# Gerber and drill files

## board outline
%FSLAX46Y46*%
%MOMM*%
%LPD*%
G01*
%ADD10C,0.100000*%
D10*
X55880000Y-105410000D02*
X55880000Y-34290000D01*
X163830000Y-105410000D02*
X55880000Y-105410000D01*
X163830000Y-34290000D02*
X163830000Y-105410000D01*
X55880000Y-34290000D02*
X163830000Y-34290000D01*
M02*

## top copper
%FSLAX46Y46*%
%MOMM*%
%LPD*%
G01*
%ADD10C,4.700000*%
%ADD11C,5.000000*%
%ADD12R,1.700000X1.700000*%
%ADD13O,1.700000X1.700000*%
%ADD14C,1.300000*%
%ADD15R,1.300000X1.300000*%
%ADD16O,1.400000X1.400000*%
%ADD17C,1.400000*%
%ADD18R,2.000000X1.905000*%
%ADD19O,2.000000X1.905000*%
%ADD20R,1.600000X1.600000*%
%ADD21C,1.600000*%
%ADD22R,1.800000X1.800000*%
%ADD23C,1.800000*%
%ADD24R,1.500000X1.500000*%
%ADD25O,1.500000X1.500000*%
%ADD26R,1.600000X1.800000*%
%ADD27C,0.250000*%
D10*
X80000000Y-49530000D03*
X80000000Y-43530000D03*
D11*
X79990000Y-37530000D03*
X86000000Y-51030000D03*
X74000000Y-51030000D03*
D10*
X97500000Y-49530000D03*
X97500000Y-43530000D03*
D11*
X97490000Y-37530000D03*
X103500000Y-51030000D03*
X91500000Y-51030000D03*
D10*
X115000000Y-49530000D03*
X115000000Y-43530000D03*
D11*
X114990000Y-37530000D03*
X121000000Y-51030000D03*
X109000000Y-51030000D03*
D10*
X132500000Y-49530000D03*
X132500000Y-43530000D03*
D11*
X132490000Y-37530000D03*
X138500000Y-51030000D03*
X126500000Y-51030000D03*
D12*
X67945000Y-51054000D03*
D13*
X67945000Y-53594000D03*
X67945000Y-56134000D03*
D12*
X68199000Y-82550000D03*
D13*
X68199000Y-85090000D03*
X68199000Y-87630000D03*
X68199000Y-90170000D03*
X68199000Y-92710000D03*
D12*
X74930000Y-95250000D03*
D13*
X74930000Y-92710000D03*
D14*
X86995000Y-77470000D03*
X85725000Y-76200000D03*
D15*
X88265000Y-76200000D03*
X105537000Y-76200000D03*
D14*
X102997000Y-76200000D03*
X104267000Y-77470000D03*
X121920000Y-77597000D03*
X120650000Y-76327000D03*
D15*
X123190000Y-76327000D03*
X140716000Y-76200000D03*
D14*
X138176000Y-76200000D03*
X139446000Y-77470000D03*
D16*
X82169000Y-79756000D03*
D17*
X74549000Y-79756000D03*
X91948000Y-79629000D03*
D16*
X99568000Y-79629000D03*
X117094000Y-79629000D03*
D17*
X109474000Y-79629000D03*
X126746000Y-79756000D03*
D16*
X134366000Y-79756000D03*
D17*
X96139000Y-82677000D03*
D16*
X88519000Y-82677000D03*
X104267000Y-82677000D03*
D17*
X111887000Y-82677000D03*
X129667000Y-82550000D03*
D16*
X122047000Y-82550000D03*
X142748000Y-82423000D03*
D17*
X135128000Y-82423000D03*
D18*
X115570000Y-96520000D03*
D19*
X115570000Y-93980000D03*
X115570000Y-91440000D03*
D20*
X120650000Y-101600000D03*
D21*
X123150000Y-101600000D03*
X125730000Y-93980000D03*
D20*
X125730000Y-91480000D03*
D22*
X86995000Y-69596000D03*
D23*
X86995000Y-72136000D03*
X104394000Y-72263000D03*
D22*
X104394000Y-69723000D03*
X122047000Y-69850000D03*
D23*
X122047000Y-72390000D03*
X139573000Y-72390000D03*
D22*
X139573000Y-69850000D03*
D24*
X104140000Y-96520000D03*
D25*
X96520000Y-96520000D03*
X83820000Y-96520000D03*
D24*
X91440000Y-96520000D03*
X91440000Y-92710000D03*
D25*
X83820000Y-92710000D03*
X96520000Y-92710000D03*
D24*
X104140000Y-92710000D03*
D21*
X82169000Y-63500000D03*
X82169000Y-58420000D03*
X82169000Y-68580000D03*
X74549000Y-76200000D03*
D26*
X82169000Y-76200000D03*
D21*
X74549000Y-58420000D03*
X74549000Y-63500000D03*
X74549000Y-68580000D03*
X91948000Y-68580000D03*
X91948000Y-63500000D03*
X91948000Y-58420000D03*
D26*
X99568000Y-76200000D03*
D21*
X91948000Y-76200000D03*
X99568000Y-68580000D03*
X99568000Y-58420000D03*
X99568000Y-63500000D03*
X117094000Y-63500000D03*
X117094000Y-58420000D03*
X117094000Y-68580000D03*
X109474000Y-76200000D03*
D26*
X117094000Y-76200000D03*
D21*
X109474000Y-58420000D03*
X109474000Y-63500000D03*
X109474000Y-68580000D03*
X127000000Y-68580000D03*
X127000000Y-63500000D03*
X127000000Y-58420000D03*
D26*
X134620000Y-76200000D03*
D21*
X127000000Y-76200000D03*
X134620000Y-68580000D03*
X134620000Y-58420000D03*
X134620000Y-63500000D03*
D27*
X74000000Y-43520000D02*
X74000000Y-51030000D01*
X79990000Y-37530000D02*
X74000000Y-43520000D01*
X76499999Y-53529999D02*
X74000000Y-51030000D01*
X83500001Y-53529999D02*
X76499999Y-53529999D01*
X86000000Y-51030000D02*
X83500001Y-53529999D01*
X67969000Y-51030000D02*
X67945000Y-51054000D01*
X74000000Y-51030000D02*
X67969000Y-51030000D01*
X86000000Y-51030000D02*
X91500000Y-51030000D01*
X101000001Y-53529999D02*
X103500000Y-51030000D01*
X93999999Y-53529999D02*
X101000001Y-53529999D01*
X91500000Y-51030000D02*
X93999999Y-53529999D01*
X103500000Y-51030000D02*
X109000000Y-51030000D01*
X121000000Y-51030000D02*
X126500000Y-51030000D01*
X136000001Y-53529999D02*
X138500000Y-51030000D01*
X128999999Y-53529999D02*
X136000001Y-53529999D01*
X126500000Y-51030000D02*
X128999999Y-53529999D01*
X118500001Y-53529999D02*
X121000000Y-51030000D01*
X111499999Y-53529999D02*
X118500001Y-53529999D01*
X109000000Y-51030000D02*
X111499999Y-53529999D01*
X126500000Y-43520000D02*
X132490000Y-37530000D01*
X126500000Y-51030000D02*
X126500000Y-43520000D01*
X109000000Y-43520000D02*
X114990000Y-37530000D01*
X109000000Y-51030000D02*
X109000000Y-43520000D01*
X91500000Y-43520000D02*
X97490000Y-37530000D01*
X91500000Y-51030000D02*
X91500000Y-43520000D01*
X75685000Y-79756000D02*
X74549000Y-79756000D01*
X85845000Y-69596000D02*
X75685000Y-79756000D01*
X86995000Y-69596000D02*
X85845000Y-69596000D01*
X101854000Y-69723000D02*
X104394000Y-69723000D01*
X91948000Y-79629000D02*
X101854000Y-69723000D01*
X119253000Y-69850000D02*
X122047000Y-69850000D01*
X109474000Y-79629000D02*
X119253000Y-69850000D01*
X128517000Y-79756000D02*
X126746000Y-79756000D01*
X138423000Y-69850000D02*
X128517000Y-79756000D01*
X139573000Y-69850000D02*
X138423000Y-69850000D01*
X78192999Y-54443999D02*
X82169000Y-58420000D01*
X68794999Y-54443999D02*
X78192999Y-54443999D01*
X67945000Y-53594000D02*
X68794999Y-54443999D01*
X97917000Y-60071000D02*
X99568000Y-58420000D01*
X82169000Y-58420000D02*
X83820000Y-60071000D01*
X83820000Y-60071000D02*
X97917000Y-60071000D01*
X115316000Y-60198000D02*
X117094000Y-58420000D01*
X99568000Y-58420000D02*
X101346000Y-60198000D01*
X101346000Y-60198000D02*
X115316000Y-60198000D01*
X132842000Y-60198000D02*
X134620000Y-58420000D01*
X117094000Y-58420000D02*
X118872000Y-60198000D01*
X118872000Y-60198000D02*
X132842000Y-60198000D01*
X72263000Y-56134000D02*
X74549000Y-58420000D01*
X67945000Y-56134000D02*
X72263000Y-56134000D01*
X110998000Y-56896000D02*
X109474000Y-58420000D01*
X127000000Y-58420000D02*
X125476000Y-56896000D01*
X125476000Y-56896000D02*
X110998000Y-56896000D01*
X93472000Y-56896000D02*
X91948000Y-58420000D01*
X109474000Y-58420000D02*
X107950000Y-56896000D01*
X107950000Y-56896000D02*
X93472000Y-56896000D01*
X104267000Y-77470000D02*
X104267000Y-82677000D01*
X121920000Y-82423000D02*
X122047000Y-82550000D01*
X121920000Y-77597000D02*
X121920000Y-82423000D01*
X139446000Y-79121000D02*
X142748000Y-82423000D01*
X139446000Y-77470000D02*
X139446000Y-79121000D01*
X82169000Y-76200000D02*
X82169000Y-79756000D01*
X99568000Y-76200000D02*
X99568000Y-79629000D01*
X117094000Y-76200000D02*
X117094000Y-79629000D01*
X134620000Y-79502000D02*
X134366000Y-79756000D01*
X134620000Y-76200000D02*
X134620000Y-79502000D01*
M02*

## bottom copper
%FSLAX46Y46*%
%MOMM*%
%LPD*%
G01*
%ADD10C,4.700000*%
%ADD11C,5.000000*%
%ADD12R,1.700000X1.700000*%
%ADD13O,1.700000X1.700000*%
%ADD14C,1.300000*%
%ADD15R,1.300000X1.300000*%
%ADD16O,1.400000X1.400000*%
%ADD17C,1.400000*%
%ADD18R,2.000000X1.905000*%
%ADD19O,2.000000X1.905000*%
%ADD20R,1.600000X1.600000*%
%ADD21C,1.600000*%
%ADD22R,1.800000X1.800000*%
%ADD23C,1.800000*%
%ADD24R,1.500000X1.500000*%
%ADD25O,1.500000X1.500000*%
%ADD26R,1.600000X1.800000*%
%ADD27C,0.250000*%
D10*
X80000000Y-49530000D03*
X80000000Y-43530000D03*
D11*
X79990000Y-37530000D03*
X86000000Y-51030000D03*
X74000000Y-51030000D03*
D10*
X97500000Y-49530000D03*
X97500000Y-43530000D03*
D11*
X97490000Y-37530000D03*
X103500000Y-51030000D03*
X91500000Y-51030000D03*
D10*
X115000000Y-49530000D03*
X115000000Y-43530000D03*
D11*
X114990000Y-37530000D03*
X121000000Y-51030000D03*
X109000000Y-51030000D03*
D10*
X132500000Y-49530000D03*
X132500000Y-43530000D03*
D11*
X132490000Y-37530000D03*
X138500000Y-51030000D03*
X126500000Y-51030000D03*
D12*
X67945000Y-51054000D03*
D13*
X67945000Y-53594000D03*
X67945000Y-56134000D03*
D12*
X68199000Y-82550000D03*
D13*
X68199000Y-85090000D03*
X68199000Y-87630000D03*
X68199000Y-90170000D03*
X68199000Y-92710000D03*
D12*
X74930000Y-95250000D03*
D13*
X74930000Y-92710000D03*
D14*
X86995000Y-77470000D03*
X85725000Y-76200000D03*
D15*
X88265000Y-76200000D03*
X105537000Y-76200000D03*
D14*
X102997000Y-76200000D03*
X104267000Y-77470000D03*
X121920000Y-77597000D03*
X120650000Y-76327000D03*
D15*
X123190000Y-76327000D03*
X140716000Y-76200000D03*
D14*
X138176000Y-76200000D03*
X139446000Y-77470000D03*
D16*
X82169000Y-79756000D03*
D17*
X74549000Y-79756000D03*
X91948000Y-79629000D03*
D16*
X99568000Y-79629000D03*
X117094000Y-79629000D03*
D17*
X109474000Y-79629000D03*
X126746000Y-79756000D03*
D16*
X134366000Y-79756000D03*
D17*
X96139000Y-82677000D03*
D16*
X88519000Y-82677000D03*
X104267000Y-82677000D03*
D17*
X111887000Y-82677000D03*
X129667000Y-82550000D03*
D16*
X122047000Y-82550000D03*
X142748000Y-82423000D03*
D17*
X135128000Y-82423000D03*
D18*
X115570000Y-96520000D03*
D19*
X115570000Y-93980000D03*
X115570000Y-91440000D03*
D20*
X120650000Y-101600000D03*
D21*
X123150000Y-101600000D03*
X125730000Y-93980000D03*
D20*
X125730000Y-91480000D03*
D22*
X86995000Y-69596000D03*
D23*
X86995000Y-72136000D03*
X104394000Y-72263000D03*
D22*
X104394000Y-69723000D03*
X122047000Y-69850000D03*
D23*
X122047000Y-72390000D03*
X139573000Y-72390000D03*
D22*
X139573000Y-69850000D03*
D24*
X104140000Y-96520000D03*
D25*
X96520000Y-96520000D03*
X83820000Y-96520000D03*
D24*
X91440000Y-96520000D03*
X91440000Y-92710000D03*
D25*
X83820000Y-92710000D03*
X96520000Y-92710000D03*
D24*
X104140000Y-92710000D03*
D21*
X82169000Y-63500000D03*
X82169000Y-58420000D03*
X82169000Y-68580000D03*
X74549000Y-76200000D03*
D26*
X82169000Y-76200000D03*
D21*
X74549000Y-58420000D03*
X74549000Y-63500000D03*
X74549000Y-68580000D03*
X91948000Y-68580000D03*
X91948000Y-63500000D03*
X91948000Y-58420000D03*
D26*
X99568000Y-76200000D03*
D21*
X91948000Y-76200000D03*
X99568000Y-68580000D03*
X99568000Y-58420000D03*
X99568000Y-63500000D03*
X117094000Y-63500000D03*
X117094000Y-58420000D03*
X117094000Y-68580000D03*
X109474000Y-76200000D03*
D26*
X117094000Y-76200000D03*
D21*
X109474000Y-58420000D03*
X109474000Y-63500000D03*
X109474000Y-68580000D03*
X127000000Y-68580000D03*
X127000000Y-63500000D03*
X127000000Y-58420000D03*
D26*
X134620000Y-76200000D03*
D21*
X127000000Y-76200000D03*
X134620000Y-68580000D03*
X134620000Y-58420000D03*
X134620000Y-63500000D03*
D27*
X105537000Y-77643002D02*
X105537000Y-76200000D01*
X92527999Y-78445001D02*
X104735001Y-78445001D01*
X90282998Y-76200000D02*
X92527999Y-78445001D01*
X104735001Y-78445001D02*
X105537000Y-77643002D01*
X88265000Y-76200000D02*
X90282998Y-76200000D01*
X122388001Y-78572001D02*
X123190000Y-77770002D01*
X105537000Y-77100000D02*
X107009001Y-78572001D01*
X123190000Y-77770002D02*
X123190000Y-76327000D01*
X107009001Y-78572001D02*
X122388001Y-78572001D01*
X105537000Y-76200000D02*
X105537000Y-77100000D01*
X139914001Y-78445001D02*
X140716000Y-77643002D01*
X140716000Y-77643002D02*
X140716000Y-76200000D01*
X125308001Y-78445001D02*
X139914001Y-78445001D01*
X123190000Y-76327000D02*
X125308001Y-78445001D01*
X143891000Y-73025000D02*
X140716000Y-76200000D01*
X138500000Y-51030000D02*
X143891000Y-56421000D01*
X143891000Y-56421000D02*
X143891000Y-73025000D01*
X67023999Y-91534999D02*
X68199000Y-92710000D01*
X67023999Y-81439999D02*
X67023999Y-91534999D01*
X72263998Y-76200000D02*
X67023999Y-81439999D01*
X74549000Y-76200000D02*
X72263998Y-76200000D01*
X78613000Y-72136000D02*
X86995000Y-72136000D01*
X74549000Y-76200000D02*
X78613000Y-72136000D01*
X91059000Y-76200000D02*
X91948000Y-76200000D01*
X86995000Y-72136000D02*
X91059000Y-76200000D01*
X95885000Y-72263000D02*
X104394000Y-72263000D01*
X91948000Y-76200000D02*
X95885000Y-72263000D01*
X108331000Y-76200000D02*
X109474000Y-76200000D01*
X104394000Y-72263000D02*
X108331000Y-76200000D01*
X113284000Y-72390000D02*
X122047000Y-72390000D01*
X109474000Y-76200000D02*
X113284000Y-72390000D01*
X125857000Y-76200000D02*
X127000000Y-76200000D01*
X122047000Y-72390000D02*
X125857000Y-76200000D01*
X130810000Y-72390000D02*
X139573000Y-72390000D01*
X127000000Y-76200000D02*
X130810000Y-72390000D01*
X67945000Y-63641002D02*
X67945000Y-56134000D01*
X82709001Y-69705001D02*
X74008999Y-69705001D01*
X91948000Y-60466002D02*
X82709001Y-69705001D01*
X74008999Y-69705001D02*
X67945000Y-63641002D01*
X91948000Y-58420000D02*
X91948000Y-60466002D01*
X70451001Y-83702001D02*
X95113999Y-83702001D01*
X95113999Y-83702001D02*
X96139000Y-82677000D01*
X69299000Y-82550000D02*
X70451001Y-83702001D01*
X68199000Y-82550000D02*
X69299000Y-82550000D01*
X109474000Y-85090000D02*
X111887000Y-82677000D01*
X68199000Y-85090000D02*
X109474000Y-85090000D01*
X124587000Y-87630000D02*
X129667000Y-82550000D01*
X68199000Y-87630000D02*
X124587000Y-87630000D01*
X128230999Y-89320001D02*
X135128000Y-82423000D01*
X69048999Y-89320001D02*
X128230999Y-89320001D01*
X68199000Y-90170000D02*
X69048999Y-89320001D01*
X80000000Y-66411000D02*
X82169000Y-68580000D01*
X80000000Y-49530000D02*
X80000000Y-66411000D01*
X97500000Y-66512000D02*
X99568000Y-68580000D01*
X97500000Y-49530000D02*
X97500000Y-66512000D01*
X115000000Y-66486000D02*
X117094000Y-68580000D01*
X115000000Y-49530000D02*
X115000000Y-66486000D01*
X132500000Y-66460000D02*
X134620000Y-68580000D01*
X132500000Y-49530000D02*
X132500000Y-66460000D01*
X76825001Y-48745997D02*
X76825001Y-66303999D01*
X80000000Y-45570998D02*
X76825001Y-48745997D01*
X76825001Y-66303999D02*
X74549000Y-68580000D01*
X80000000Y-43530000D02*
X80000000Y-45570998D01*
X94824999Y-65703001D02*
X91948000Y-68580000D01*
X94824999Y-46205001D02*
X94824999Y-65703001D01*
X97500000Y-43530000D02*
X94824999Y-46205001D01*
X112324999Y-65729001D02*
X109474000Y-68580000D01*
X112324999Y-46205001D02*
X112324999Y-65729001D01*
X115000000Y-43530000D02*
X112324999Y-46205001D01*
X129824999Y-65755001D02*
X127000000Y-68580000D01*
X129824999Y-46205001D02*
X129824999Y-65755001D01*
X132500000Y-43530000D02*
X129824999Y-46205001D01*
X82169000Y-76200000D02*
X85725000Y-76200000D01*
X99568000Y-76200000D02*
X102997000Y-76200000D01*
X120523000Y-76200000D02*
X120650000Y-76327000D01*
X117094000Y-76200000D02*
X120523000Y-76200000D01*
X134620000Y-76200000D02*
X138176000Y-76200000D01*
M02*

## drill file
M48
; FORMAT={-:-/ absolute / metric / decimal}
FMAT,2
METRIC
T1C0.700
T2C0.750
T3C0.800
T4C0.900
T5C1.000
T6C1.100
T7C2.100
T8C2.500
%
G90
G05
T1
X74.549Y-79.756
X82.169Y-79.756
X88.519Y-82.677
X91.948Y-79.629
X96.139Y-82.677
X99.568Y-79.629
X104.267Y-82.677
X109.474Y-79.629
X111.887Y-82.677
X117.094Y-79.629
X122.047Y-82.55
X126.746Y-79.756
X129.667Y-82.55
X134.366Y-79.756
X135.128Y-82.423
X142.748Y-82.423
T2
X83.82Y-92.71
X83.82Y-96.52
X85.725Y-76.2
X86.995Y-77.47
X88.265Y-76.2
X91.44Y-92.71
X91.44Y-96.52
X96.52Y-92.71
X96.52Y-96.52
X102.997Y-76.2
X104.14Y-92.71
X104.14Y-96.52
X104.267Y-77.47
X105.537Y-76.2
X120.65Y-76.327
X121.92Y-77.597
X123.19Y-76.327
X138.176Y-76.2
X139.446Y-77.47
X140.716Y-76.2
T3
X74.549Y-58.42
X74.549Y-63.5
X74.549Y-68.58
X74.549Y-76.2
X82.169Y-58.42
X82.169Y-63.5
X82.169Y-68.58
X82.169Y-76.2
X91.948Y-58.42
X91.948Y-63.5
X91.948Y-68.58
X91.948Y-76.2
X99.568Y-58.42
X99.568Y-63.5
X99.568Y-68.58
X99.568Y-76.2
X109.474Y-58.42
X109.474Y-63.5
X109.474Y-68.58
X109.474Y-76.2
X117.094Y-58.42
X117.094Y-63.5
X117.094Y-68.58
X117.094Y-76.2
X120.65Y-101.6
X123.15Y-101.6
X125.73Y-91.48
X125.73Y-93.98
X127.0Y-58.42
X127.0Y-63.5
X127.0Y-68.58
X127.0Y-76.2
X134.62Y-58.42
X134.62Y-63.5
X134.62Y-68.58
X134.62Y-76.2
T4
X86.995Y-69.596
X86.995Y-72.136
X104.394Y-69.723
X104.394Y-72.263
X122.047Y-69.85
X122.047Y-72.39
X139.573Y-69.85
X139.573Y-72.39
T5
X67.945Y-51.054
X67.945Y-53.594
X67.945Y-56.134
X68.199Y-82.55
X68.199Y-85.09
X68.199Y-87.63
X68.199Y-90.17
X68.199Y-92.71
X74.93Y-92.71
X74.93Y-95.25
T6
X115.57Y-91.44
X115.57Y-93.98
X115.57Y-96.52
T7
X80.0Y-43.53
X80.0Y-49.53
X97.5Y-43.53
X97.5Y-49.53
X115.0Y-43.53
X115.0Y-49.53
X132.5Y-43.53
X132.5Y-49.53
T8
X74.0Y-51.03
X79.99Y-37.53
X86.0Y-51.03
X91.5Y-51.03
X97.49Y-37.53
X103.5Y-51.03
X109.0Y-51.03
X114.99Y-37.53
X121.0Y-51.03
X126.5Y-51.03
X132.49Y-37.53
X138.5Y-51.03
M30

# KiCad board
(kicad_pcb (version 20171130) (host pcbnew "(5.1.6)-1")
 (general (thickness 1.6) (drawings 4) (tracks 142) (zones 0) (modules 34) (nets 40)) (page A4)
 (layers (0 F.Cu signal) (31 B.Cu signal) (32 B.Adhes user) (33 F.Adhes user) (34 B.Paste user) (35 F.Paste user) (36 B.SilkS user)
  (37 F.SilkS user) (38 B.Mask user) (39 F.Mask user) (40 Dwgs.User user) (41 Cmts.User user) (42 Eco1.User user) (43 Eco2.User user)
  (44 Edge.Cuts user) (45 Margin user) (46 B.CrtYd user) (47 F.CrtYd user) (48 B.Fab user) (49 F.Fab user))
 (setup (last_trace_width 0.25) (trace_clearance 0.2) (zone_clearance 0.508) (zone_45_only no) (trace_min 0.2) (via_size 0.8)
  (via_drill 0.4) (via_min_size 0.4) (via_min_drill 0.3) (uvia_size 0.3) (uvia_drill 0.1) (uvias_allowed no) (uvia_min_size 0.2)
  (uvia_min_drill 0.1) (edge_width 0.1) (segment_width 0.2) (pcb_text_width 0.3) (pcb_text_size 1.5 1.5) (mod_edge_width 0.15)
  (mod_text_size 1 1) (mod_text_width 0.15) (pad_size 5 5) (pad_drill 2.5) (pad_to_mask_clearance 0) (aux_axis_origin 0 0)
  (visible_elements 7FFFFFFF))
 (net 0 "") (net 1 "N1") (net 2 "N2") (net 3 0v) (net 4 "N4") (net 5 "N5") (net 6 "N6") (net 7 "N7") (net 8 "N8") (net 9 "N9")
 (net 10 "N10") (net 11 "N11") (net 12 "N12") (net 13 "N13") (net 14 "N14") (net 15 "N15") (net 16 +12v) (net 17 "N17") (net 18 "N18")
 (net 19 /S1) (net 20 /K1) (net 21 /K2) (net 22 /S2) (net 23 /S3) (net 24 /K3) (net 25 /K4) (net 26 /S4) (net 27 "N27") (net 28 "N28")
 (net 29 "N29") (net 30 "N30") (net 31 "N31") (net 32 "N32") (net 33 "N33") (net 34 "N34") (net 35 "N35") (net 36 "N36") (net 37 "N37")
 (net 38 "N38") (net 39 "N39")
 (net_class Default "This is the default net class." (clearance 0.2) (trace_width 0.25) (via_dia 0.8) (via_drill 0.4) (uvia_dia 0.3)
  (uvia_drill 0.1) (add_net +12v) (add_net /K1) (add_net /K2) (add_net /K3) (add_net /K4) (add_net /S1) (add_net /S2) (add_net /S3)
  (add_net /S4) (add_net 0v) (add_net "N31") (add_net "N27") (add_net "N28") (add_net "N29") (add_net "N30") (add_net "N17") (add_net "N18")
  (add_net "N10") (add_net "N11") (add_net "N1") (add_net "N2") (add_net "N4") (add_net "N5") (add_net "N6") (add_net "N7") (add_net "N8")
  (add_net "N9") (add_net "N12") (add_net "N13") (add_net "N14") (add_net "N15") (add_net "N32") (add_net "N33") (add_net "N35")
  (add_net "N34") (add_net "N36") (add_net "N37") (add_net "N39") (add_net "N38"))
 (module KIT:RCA (layer F.Cu) (at 80 49.53 270)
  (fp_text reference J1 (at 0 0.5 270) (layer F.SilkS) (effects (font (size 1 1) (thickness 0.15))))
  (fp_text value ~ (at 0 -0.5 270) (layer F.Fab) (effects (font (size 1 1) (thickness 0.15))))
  (pad 1 thru_hole circle (at 0 0 270) (size 4.7 4.7) (drill 2.1) (layers *.Cu *.Mask) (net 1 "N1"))
  (pad 3 thru_hole circle (at -6 0 270) (size 4.7 4.7) (drill 2.1) (layers *.Cu *.Mask) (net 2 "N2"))
  (pad 2 thru_hole circle (at -12 0.01 270) (size 5 5) (drill 2.5) (layers *.Cu *.Mask) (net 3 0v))
  (pad 2 thru_hole circle (at 1.5 -6 270) (size 5 5) (drill 2.5) (layers *.Cu *.Mask) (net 3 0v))
  (pad 2 thru_hole circle (at 1.5 6 270) (size 5 5) (drill 2.5) (layers *.Cu *.Mask) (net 3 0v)))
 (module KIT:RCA (layer F.Cu) (at 97.5 49.53 270)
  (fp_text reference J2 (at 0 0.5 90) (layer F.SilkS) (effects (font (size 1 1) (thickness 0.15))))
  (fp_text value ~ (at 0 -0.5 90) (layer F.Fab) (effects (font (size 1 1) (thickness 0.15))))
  (pad 1 thru_hole circle (at 0 0 270) (size 4.7 4.7) (drill 2.1) (layers *.Cu *.Mask) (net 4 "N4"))
  (pad 3 thru_hole circle (at -6 0 270) (size 4.7 4.7) (drill 2.1) (layers *.Cu *.Mask) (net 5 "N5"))
  (pad 2 thru_hole circle (at -12 0.01 270) (size 5 5) (drill 2.5) (layers *.Cu *.Mask) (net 3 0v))
  (pad 2 thru_hole circle (at 1.5 -6 270) (size 5 5) (drill 2.5) (layers *.Cu *.Mask) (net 3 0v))
  (pad 2 thru_hole circle (at 1.5 6 270) (size 5 5) (drill 2.5) (layers *.Cu *.Mask) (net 3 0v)))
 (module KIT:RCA (layer F.Cu) (at 115 49.53 270)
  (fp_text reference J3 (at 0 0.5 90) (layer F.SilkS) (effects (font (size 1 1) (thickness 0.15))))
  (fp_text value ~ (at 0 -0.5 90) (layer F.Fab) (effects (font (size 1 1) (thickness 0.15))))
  (pad 1 thru_hole circle (at 0 0 270) (size 4.7 4.7) (drill 2.1) (layers *.Cu *.Mask) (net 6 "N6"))
  (pad 3 thru_hole circle (at -6 0 270) (size 4.7 4.7) (drill 2.1) (layers *.Cu *.Mask) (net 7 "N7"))
  (pad 2 thru_hole circle (at -12 0.01 270) (size 5 5) (drill 2.5) (layers *.Cu *.Mask) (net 3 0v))
  (pad 2 thru_hole circle (at 1.5 -6 270) (size 5 5) (drill 2.5) (layers *.Cu *.Mask) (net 3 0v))
  (pad 2 thru_hole circle (at 1.5 6 270) (size 5 5) (drill 2.5) (layers *.Cu *.Mask) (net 3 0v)))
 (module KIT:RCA (layer F.Cu) (at 132.5 49.53 270)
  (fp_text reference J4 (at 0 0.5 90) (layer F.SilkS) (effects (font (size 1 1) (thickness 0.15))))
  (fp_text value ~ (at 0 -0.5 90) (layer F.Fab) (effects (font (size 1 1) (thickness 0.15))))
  (pad 1 thru_hole circle (at 0 0 270) (size 4.7 4.7) (drill 2.1) (layers *.Cu *.Mask) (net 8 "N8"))
  (pad 3 thru_hole circle (at -6 0 270) (size 4.7 4.7) (drill 2.1) (layers *.Cu *.Mask) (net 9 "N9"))
  (pad 2 thru_hole circle (at -12 0.01 270) (size 5 5) (drill 2.5) (layers *.Cu *.Mask) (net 3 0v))
  (pad 2 thru_hole circle (at 1.5 -6 270) (size 5 5) (drill 2.5) (layers *.Cu *.Mask) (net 3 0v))
  (pad 2 thru_hole circle (at 1.5 6 270) (size 5 5) (drill 2.5) (layers *.Cu *.Mask) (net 3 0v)))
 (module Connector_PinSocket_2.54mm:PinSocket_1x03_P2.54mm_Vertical (layer F.Cu) (at 67.945 51.054)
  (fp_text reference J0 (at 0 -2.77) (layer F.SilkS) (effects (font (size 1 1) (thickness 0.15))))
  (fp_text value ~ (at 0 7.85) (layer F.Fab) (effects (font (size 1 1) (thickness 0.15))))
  (pad 1 thru_hole rect (at 0 0) (size 1.7 1.7) (drill 1) (layers *.Cu *.Mask) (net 3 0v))
  (pad 2 thru_hole oval (at 0 2.54) (size 1.7 1.7) (drill 1) (layers *.Cu *.Mask) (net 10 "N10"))
  (pad 3 thru_hole oval (at 0 5.08) (size 1.7 1.7) (drill 1) (layers *.Cu *.Mask) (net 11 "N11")))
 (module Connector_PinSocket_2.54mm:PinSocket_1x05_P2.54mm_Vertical (layer F.Cu) (at 68.199 82.55)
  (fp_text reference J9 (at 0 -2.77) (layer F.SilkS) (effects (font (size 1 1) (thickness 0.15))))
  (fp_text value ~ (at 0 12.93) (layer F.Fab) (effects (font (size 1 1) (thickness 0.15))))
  (pad 1 thru_hole rect (at 0 0) (size 1.7 1.7) (drill 1) (layers *.Cu *.Mask) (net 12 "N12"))
  (pad 2 thru_hole oval (at 0 2.54) (size 1.7 1.7) (drill 1) (layers *.Cu *.Mask) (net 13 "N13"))
  (pad 3 thru_hole oval (at 0 5.08) (size 1.7 1.7) (drill 1) (layers *.Cu *.Mask) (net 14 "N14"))
  (pad 4 thru_hole oval (at 0 7.62) (size 1.7 1.7) (drill 1) (layers *.Cu *.Mask) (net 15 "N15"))
  (pad 5 thru_hole oval (at 0 10.16) (size 1.7 1.7) (drill 1) (layers *.Cu *.Mask) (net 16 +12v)))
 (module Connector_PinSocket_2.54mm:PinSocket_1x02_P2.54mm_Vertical (layer F.Cu) (at 74.93 95.25 180)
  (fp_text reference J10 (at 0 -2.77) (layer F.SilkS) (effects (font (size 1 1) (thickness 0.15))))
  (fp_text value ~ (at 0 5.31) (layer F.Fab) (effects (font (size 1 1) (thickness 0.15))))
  (pad 1 thru_hole rect (at 0 0 180) (size 1.7 1.7) (drill 1) (layers *.Cu *.Mask) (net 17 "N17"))
  (pad 2 thru_hole oval (at 0 2.54 180) (size 1.7 1.7) (drill 1) (layers *.Cu *.Mask) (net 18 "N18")))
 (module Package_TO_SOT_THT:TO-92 (layer F.Cu) (at 88.265 76.2 180)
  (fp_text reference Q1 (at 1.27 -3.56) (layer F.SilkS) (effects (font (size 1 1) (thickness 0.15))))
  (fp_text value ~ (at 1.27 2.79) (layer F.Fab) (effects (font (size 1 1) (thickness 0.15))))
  (pad 2 thru_hole circle (at 1.27 -1.27 270) (size 1.3 1.3) (drill 0.75) (layers *.Cu *.Mask) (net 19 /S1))
  (pad 3 thru_hole circle (at 2.54 0 270) (size 1.3 1.3) (drill 0.75) (layers *.Cu *.Mask) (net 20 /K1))
  (pad 1 thru_hole rect (at 0 0 270) (size 1.3 1.3) (drill 0.75) (layers *.Cu *.Mask) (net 3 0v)))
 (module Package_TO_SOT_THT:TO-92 (layer F.Cu) (at 105.537 76.2 180)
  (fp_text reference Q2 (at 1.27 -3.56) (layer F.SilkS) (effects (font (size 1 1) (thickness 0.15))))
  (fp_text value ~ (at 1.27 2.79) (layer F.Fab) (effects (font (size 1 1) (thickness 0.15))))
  (pad 1 thru_hole rect (at 0 0 270) (size 1.3 1.3) (drill 0.75) (layers *.Cu *.Mask) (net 3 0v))
  (pad 3 thru_hole circle (at 2.54 0 270) (size 1.3 1.3) (drill 0.75) (layers *.Cu *.Mask) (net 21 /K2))
  (pad 2 thru_hole circle (at 1.27 -1.27 270) (size 1.3 1.3) (drill 0.75) (layers *.Cu *.Mask) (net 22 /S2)))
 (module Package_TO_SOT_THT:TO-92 (layer F.Cu) (at 123.19 76.327 180)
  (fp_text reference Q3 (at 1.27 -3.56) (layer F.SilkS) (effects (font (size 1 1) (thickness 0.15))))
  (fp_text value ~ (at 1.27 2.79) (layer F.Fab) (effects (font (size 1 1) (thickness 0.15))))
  (pad 2 thru_hole circle (at 1.27 -1.27 270) (size 1.3 1.3) (drill 0.75) (layers *.Cu *.Mask) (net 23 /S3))
  (pad 3 thru_hole circle (at 2.54 0 270) (size 1.3 1.3) (drill 0.75) (layers *.Cu *.Mask) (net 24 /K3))
  (pad 1 thru_hole rect (at 0 0 270) (size 1.3 1.3) (drill 0.75) (layers *.Cu *.Mask) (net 3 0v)))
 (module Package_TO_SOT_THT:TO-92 (layer F.Cu) (at 140.716 76.2 180)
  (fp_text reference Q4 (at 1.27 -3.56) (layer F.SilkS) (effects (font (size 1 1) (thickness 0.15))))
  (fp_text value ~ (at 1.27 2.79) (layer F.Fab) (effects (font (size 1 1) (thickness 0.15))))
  (pad 1 thru_hole rect (at 0 0 270) (size 1.3 1.3) (drill 0.75) (layers *.Cu *.Mask) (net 3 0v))
  (pad 3 thru_hole circle (at 2.54 0 270) (size 1.3 1.3) (drill 0.75) (layers *.Cu *.Mask) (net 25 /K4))
  (pad 2 thru_hole circle (at 1.27 -1.27 270) (size 1.3 1.3) (drill 0.75) (layers *.Cu *.Mask) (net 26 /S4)))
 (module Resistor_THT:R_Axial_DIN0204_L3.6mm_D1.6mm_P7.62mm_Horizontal (layer F.Cu) (at 74.549 79.756)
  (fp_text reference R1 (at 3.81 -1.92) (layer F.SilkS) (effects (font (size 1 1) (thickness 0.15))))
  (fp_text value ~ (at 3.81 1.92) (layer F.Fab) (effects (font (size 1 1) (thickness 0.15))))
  (pad 2 thru_hole oval (at 7.62 0) (size 1.4 1.4) (drill 0.7) (layers *.Cu *.Mask) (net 20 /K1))
  (pad 1 thru_hole circle (at 0 0) (size 1.4 1.4) (drill 0.7) (layers *.Cu *.Mask) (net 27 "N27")))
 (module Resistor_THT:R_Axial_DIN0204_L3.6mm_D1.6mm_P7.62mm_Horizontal (layer F.Cu) (at 91.948 79.629)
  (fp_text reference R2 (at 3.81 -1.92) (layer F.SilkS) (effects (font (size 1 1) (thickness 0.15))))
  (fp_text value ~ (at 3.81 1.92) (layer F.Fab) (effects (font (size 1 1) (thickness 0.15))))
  (pad 1 thru_hole circle (at 0 0) (size 1.4 1.4) (drill 0.7) (layers *.Cu *.Mask) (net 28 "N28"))
  (pad 2 thru_hole oval (at 7.62 0) (size 1.4 1.4) (drill 0.7) (layers *.Cu *.Mask) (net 21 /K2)))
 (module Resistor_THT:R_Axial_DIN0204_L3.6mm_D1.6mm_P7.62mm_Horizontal (layer F.Cu) (at 109.474 79.629)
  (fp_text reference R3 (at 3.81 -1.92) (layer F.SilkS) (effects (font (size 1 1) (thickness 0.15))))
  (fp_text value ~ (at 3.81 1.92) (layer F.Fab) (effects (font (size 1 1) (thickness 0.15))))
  (pad 2 thru_hole oval (at 7.62 0) (size 1.4 1.4) (drill 0.7) (layers *.Cu *.Mask) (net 24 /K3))
  (pad 1 thru_hole circle (at 0 0) (size 1.4 1.4) (drill 0.7) (layers *.Cu *.Mask) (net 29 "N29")))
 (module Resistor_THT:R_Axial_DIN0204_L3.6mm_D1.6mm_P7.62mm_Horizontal (layer F.Cu) (at 126.746 79.756)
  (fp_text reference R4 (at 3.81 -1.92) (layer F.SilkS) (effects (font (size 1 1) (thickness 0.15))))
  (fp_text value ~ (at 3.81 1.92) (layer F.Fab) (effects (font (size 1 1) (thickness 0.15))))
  (pad 1 thru_hole circle (at 0 0) (size 1.4 1.4) (drill 0.7) (layers *.Cu *.Mask) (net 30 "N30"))
  (pad 2 thru_hole oval (at 7.62 0) (size 1.4 1.4) (drill 0.7) (layers *.Cu *.Mask) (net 25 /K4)))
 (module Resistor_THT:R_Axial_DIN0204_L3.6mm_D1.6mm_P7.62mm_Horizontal (layer F.Cu) (at 96.139 82.677 180)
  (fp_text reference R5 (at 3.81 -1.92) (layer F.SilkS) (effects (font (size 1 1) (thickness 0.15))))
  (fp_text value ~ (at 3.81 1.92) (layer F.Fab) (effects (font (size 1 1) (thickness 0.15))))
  (pad 1 thru_hole circle (at 0 0 180) (size 1.4 1.4) (drill 0.7) (layers *.Cu *.Mask) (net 12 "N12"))
  (pad 2 thru_hole oval (at 7.62 0 180) (size 1.4 1.4) (drill 0.7) (layers *.Cu *.Mask) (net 19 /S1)))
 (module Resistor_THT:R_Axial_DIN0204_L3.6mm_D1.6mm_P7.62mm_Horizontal (layer F.Cu) (at 111.887 82.677 180)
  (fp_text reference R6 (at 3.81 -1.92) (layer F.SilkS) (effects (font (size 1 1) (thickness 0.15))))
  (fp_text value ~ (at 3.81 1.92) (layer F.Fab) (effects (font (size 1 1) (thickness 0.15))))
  (pad 2 thru_hole oval (at 7.62 0 180) (size 1.4 1.4) (drill 0.7) (layers *.Cu *.Mask) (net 22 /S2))
  (pad 1 thru_hole circle (at 0 0 180) (size 1.4 1.4) (drill 0.7) (layers *.Cu *.Mask) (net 13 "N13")))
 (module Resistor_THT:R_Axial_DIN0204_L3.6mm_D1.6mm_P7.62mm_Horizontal (layer F.Cu) (at 129.667 82.55 180)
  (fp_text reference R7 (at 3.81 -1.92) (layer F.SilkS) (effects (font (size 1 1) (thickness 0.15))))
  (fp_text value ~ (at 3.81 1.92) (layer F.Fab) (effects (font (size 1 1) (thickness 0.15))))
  (pad 1 thru_hole circle (at 0 0 180) (size 1.4 1.4) (drill 0.7) (layers *.Cu *.Mask) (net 14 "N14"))
  (pad 2 thru_hole oval (at 7.62 0 180) (size 1.4 1.4) (drill 0.7) (layers *.Cu *.Mask) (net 23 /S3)))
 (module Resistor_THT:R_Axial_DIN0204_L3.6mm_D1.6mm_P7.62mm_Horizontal (layer F.Cu) (at 135.128 82.423)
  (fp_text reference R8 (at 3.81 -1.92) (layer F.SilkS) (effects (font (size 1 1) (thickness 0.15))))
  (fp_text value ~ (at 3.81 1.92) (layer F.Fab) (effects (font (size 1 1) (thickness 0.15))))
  (pad 2 thru_hole oval (at 7.62 0) (size 1.4 1.4) (drill 0.7) (layers *.Cu *.Mask) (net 26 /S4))
  (pad 1 thru_hole circle (at 0 0) (size 1.4 1.4) (drill 0.7) (layers *.Cu *.Mask) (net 15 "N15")))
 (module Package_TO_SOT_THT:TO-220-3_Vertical (layer F.Cu) (at 115.57 96.52 90)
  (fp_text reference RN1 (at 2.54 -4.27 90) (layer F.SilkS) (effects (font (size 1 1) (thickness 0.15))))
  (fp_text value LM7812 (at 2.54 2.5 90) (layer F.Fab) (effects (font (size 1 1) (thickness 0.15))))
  (pad 1 thru_hole rect (at 0 0 90) (size 1.905 2) (drill 1.1) (layers *.Cu *.Mask) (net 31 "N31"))
  (pad 2 thru_hole oval (at 2.54 0 90) (size 1.905 2) (drill 1.1) (layers *.Cu *.Mask) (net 3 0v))
  (pad 3 thru_hole oval (at 5.08 0 90) (size 1.905 2) (drill 1.1) (layers *.Cu *.Mask) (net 16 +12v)))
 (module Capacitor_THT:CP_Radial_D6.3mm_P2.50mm (layer F.Cu) (at 120.65 101.6)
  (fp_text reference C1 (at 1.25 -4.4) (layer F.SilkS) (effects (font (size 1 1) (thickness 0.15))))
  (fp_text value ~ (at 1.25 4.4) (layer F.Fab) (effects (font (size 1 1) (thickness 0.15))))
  (pad 1 thru_hole rect (at 0 0) (size 1.6 1.6) (drill 0.8) (layers *.Cu *.Mask) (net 31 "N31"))
  (pad 2 thru_hole circle (at 2.5 0) (size 1.6 1.6) (drill 0.8) (layers *.Cu *.Mask) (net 3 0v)))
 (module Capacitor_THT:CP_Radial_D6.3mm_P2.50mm (layer F.Cu) (at 125.73 91.48 270)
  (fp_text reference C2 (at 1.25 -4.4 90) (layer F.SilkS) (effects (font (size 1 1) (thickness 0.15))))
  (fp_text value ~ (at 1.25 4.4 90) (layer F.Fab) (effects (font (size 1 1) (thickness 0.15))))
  (pad 2 thru_hole circle (at 2.5 0 270) (size 1.6 1.6) (drill 0.8) (layers *.Cu *.Mask) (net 3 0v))
  (pad 1 thru_hole rect (at 0 0 270) (size 1.6 1.6) (drill 0.8) (layers *.Cu *.Mask) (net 16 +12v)))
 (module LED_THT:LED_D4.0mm (layer F.Cu) (at 86.995 69.596 270)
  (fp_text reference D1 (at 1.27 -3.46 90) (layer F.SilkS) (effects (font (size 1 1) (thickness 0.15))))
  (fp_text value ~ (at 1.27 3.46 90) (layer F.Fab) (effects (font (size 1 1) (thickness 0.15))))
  (pad 1 thru_hole rect (at 0 0 270) (size 1.8 1.8) (drill 0.9) (layers *.Cu *.Mask) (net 27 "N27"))
  (pad 2 thru_hole circle (at 2.54 0 270) (size 1.8 1.8) (drill 0.9) (layers *.Cu *.Mask) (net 16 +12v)))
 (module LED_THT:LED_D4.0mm (layer F.Cu) (at 104.394 69.723 270)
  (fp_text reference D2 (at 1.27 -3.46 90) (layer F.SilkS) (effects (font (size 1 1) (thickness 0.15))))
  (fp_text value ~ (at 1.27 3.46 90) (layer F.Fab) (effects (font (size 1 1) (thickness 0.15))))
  (pad 2 thru_hole circle (at 2.54 0 270) (size 1.8 1.8) (drill 0.9) (layers *.Cu *.Mask) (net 16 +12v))
  (pad 1 thru_hole rect (at 0 0 270) (size 1.8 1.8) (drill 0.9) (layers *.Cu *.Mask) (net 28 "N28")))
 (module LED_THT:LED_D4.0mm (layer F.Cu) (at 122.047 69.85 270)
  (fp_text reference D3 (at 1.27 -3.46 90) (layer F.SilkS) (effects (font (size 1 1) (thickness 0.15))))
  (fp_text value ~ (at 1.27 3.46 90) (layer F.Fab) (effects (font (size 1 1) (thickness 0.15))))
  (pad 1 thru_hole rect (at 0 0 270) (size 1.8 1.8) (drill 0.9) (layers *.Cu *.Mask) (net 29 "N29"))
  (pad 2 thru_hole circle (at 2.54 0 270) (size 1.8 1.8) (drill 0.9) (layers *.Cu *.Mask) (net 16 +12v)))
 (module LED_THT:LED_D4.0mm (layer F.Cu) (at 139.573 69.85 270)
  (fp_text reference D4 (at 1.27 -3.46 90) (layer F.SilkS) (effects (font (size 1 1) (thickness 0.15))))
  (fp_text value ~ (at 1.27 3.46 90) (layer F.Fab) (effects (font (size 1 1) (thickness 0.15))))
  (pad 2 thru_hole circle (at 2.54 0 270) (size 1.8 1.8) (drill 0.9) (layers *.Cu *.Mask) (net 16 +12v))
  (pad 1 thru_hole rect (at 0 0 270) (size 1.8 1.8) (drill 0.9) (layers *.Cu *.Mask) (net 30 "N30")))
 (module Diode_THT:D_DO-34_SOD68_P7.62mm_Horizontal (layer F.Cu) (at 104.14 96.52 180)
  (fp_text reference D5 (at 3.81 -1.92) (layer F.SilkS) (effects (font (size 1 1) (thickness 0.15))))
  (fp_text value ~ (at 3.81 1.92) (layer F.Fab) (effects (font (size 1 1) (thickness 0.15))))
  (pad 1 thru_hole rect (at 0 0 180) (size 1.5 1.5) (drill 0.75) (layers *.Cu *.Mask) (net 31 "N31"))
  (pad 2 thru_hole oval (at 7.62 0 180) (size 1.5 1.5) (drill 0.75) (layers *.Cu *.Mask) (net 17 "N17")))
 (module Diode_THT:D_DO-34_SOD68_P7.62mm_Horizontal (layer F.Cu) (at 91.44 96.52 180)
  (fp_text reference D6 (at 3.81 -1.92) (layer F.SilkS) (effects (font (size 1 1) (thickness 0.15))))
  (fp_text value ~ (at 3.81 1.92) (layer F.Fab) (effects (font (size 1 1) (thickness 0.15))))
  (pad 2 thru_hole oval (at 7.62 0 180) (size 1.5 1.5) (drill 0.75) (layers *.Cu *.Mask) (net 3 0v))
  (pad 1 thru_hole rect (at 0 0 180) (size 1.5 1.5) (drill 0.75) (layers *.Cu *.Mask) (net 17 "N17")))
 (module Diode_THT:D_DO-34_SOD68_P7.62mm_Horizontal (layer F.Cu) (at 91.44 92.71 180)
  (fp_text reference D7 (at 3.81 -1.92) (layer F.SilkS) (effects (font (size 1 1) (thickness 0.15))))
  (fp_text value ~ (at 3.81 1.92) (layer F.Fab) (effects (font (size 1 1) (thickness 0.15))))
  (pad 1 thru_hole rect (at 0 0 180) (size 1.5 1.5) (drill 0.75) (layers *.Cu *.Mask) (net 18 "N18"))
  (pad 2 thru_hole oval (at 7.62 0 180) (size 1.5 1.5) (drill 0.75) (layers *.Cu *.Mask) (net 3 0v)))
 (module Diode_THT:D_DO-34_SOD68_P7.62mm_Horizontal (layer F.Cu) (at 104.14 92.71 180)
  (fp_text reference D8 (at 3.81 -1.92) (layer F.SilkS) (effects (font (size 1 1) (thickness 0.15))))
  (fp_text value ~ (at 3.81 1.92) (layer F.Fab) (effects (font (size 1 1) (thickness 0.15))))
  (pad 2 thru_hole oval (at 7.62 0 180) (size 1.5 1.5) (drill 0.75) (layers *.Cu *.Mask) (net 18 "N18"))
  (pad 1 thru_hole rect (at 0 0 180) (size 1.5 1.5) (drill 0.75) (layers *.Cu *.Mask) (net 31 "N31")))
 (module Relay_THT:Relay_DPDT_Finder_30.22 (layer F.Cu) (at 82.169 76.2 90)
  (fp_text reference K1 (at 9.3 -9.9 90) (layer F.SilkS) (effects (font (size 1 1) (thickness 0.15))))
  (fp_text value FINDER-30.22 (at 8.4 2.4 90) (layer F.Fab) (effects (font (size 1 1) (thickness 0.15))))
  (pad 12 thru_hole circle (at 12.7 0 180) (size 1.6 1.6) (drill 0.8) (layers *.Cu *.Mask) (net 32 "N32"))
  (pad 14 thru_hole circle (at 17.78 0 180) (size 1.6 1.6) (drill 0.8) (layers *.Cu *.Mask) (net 10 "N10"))
  (pad 11 thru_hole circle (at 7.62 0 180) (size 1.6 1.6) (drill 0.8) (layers *.Cu *.Mask) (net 1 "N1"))
  (pad A2 thru_hole circle (at 0 -7.62 180) (size 1.6 1.6) (drill 0.8) (layers *.Cu *.Mask) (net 16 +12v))
  (pad A1 thru_hole rect (at 0 0 180) (size 1.6 1.8) (drill 0.8) (layers *.Cu *.Mask) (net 20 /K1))
  (pad 24 thru_hole circle (at 17.78 -7.62 270) (size 1.6 1.6) (drill 0.8) (layers *.Cu *.Mask) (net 11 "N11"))
  (pad 22 thru_hole circle (at 12.7 -7.62 180) (size 1.6 1.6) (drill 0.8) (layers *.Cu *.Mask) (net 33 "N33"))
  (pad 21 thru_hole circle (at 7.62 -7.62 180) (size 1.6 1.6) (drill 0.8) (layers *.Cu *.Mask) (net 2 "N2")))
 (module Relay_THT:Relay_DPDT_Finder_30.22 (layer F.Cu) (at 99.568 76.2 90)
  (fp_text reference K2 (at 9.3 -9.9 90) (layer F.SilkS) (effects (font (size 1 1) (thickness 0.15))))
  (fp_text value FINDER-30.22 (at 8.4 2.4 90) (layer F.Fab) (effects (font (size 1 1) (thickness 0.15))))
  (pad 21 thru_hole circle (at 7.62 -7.62 180) (size 1.6 1.6) (drill 0.8) (layers *.Cu *.Mask) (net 5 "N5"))
  (pad 22 thru_hole circle (at 12.7 -7.62 180) (size 1.6 1.6) (drill 0.8) (layers *.Cu *.Mask) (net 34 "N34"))
  (pad 24 thru_hole circle (at 17.78 -7.62 270) (size 1.6 1.6) (drill 0.8) (layers *.Cu *.Mask) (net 11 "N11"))
  (pad A1 thru_hole rect (at 0 0 180) (size 1.6 1.8) (drill 0.8) (layers *.Cu *.Mask) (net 21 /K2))
  (pad A2 thru_hole circle (at 0 -7.62 180) (size 1.6 1.6) (drill 0.8) (layers *.Cu *.Mask) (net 16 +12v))
  (pad 11 thru_hole circle (at 7.62 0 180) (size 1.6 1.6) (drill 0.8) (layers *.Cu *.Mask) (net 4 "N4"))
  (pad 14 thru_hole circle (at 17.78 0 180) (size 1.6 1.6) (drill 0.8) (layers *.Cu *.Mask) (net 10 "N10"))
  (pad 12 thru_hole circle (at 12.7 0 180) (size 1.6 1.6) (drill 0.8) (layers *.Cu *.Mask) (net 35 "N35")))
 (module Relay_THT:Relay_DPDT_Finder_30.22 (layer F.Cu) (at 117.094 76.2 90)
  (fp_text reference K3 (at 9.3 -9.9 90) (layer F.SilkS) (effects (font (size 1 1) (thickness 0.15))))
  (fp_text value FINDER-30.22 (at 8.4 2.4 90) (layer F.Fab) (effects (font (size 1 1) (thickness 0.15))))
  (pad 12 thru_hole circle (at 12.7 0 180) (size 1.6 1.6) (drill 0.8) (layers *.Cu *.Mask) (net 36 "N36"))
  (pad 14 thru_hole circle (at 17.78 0 180) (size 1.6 1.6) (drill 0.8) (layers *.Cu *.Mask) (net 10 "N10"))
  (pad 11 thru_hole circle (at 7.62 0 180) (size 1.6 1.6) (drill 0.8) (layers *.Cu *.Mask) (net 6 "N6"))
  (pad A2 thru_hole circle (at 0 -7.62 180) (size 1.6 1.6) (drill 0.8) (layers *.Cu *.Mask) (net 16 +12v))
  (pad A1 thru_hole rect (at 0 0 180) (size 1.6 1.8) (drill 0.8) (layers *.Cu *.Mask) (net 24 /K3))
  (pad 24 thru_hole circle (at 17.78 -7.62 270) (size 1.6 1.6) (drill 0.8) (layers *.Cu *.Mask) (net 11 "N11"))
  (pad 22 thru_hole circle (at 12.7 -7.62 180) (size 1.6 1.6) (drill 0.8) (layers *.Cu *.Mask) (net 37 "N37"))
  (pad 21 thru_hole circle (at 7.62 -7.62 180) (size 1.6 1.6) (drill 0.8) (layers *.Cu *.Mask) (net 7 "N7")))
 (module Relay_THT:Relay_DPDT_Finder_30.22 (layer F.Cu) (at 134.62 76.2 90)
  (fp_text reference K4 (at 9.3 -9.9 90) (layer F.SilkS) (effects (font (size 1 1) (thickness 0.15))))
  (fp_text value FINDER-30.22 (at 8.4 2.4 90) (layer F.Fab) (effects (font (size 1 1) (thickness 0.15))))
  (pad 21 thru_hole circle (at 7.62 -7.62 180) (size 1.6 1.6) (drill 0.8) (layers *.Cu *.Mask) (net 9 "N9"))
  (pad 22 thru_hole circle (at 12.7 -7.62 180) (size 1.6 1.6) (drill 0.8) (layers *.Cu *.Mask) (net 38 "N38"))
  (pad 24 thru_hole circle (at 17.78 -7.62 270) (size 1.6 1.6) (drill 0.8) (layers *.Cu *.Mask) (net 11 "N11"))
  (pad A1 thru_hole rect (at 0 0 180) (size 1.6 1.8) (drill 0.8) (layers *.Cu *.Mask) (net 25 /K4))
  (pad A2 thru_hole circle (at 0 -7.62 180) (size 1.6 1.6) (drill 0.8) (layers *.Cu *.Mask) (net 16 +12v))
  (pad 11 thru_hole circle (at 7.62 0 180) (size 1.6 1.6) (drill 0.8) (layers *.Cu *.Mask) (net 8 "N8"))
  (pad 14 thru_hole circle (at 17.78 0 180) (size 1.6 1.6) (drill 0.8) (layers *.Cu *.Mask) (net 10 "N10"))
  (pad 12 thru_hole circle (at 12.7 0 180) (size 1.6 1.6) (drill 0.8) (layers *.Cu *.Mask) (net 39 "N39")))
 (gr_line (start 55.88 105.41) (end 55.88 34.29) (layer Edge.Cuts) (width 0.1))
 (gr_line (start 163.83 105.41) (end 55.88 105.41) (layer Edge.Cuts) (width 0.1))
 (gr_line (start 163.83 34.29) (end 163.83 105.41) (layer Edge.Cuts) (width 0.1))
 (gr_line (start 55.88 34.29) (end 163.83 34.29) (layer Edge.Cuts) (width 0.1))
 (segment (start 74 43.52) (end 74 51.03) (width 0.25) (layer F.Cu) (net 3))
 (segment (start 79.99 37.53) (end 74 43.52) (width 0.25) (layer F.Cu) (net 3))
 (segment (start 76.499999 53.529999) (end 74 51.03) (width 0.25) (layer F.Cu) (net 3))
 (segment (start 83.500001 53.529999) (end 76.499999 53.529999) (width 0.25) (layer F.Cu) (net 3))
 (segment (start 86 51.03) (end 83.500001 53.529999) (width 0.25) (layer F.Cu) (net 3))
 (segment (start 67.969 51.03) (end 67.945 51.054) (width 0.25) (layer F.Cu) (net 3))
 (segment (start 74 51.03) (end 67.969 51.03) (width 0.25) (layer F.Cu) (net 3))
 (segment (start 86 51.03) (end 91.5 51.03) (width 0.25) (layer F.Cu) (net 3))
 (segment (start 101.000001 53.529999) (end 103.5 51.03) (width 0.25) (layer F.Cu) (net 3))
 (segment (start 93.999999 53.529999) (end 101.000001 53.529999) (width 0.25) (layer F.Cu) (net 3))
 (segment (start 91.5 51.03) (end 93.999999 53.529999) (width 0.25) (layer F.Cu) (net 3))
 (segment (start 103.5 51.03) (end 109 51.03) (width 0.25) (layer F.Cu) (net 3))
 (segment (start 121 51.03) (end 126.5 51.03) (width 0.25) (layer F.Cu) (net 3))
 (segment (start 136.000001 53.529999) (end 138.5 51.03) (width 0.25) (layer F.Cu) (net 3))
 (segment (start 128.999999 53.529999) (end 136.000001 53.529999) (width 0.25) (layer F.Cu) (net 3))
 (segment (start 126.5 51.03) (end 128.999999 53.529999) (width 0.25) (layer F.Cu) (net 3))
 (segment (start 118.500001 53.529999) (end 121 51.03) (width 0.25) (layer F.Cu) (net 3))
 (segment (start 111.499999 53.529999) (end 118.500001 53.529999) (width 0.25) (layer F.Cu) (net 3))
 (segment (start 109 51.03) (end 111.499999 53.529999) (width 0.25) (layer F.Cu) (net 3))
 (segment (start 126.5 43.52) (end 132.49 37.53) (width 0.25) (layer F.Cu) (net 3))
 (segment (start 126.5 51.03) (end 126.5 43.52) (width 0.25) (layer F.Cu) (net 3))
 (segment (start 109 43.52) (end 114.99 37.53) (width 0.25) (layer F.Cu) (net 3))
 (segment (start 109 51.03) (end 109 43.52) (width 0.25) (layer F.Cu) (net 3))
 (segment (start 91.5 43.52) (end 97.49 37.53) (width 0.25) (layer F.Cu) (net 3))
 (segment (start 91.5 51.03) (end 91.5 43.52) (width 0.25) (layer F.Cu) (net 3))
 (segment (start 105.537 77.643002) (end 105.537 76.2) (width 0.25) (layer B.Cu) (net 3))
 (segment (start 92.527999 78.445001) (end 104.735001 78.445001) (width 0.25) (layer B.Cu) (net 3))
 (segment (start 90.282998 76.2) (end 92.527999 78.445001) (width 0.25) (layer B.Cu) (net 3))
 (segment (start 104.735001 78.445001) (end 105.537 77.643002) (width 0.25) (layer B.Cu) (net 3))
 (segment (start 88.265 76.2) (end 90.282998 76.2) (width 0.25) (layer B.Cu) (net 3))
 (segment (start 122.388001 78.572001) (end 123.19 77.770002) (width 0.25) (layer B.Cu) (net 3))
 (segment (start 105.537 77.1) (end 107.009001 78.572001) (width 0.25) (layer B.Cu) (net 3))
 (segment (start 123.19 77.770002) (end 123.19 76.327) (width 0.25) (layer B.Cu) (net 3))
 (segment (start 107.009001 78.572001) (end 122.388001 78.572001) (width 0.25) (layer B.Cu) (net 3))
 (segment (start 105.537 76.2) (end 105.537 77.1) (width 0.25) (layer B.Cu) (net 3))
 (segment (start 139.914001 78.445001) (end 140.716 77.643002) (width 0.25) (layer B.Cu) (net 3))
 (segment (start 140.716 77.643002) (end 140.716 76.2) (width 0.25) (layer B.Cu) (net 3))
 (segment (start 125.308001 78.445001) (end 139.914001 78.445001) (width 0.25) (layer B.Cu) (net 3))
 (segment (start 123.19 76.327) (end 125.308001 78.445001) (width 0.25) (layer B.Cu) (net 3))
 (segment (start 143.891 73.025) (end 140.716 76.2) (width 0.25) (layer B.Cu) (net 3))
 (segment (start 138.5 51.03) (end 143.891 56.421) (width 0.25) (layer B.Cu) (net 3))
 (segment (start 143.891 56.421) (end 143.891 73.025) (width 0.25) (layer B.Cu) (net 3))
 (segment (start 67.023999 91.534999) (end 68.199 92.71) (width 0.25) (layer B.Cu) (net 16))
 (segment (start 67.023999 81.439999) (end 67.023999 91.534999) (width 0.25) (layer B.Cu) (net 16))
 (segment (start 72.263998 76.2) (end 67.023999 81.439999) (width 0.25) (layer B.Cu) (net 16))
 (segment (start 74.549 76.2) (end 72.263998 76.2) (width 0.25) (layer B.Cu) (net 16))
 (segment (start 78.613 72.136) (end 86.995 72.136) (width 0.25) (layer B.Cu) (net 16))
 (segment (start 74.549 76.2) (end 78.613 72.136) (width 0.25) (layer B.Cu) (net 16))
 (segment (start 91.059 76.2) (end 91.948 76.2) (width 0.25) (layer B.Cu) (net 16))
 (segment (start 86.995 72.136) (end 91.059 76.2) (width 0.25) (layer B.Cu) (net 16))
 (segment (start 95.885 72.263) (end 104.394 72.263) (width 0.25) (layer B.Cu) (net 16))
 (segment (start 91.948 76.2) (end 95.885 72.263) (width 0.25) (layer B.Cu) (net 16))
 (segment (start 108.331 76.2) (end 109.474 76.2) (width 0.25) (layer B.Cu) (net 16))
 (segment (start 104.394 72.263) (end 108.331 76.2) (width 0.25) (layer B.Cu) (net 16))
 (segment (start 113.284 72.39) (end 122.047 72.39) (width 0.25) (layer B.Cu) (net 16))
 (segment (start 109.474 76.2) (end 113.284 72.39) (width 0.25) (layer B.Cu) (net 16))
 (segment (start 125.857 76.2) (end 127 76.2) (width 0.25) (layer B.Cu) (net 16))
 (segment (start 122.047 72.39) (end 125.857 76.2) (width 0.25) (layer B.Cu) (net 16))
 (segment (start 130.81 72.39) (end 139.573 72.39) (width 0.25) (layer B.Cu) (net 16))
 (segment (start 127 76.2) (end 130.81 72.39) (width 0.25) (layer B.Cu) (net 16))
 (segment (start 75.685 79.756) (end 74.549 79.756) (width 0.25) (layer F.Cu) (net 27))
 (segment (start 85.845 69.596) (end 75.685 79.756) (width 0.25) (layer F.Cu) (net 27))
 (segment (start 86.995 69.596) (end 85.845 69.596) (width 0.25) (layer F.Cu) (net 27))
 (segment (start 101.854 69.723) (end 104.394 69.723) (width 0.25) (layer F.Cu) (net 28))
 (segment (start 91.948 79.629) (end 101.854 69.723) (width 0.25) (layer F.Cu) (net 28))
 (segment (start 119.253 69.85) (end 122.047 69.85) (width 0.25) (layer F.Cu) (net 29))
 (segment (start 109.474 79.629) (end 119.253 69.85) (width 0.25) (layer F.Cu) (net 29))
 (segment (start 128.517 79.756) (end 126.746 79.756) (width 0.25) (layer F.Cu) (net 30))
 (segment (start 138.423 69.85) (end 128.517 79.756) (width 0.25) (layer F.Cu) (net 30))
 (segment (start 139.573 69.85) (end 138.423 69.85) (width 0.25) (layer F.Cu) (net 30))
 (segment (start 78.192999 54.443999) (end 82.169 58.42) (width 0.25) (layer F.Cu) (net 10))
 (segment (start 68.794999 54.443999) (end 78.192999 54.443999) (width 0.25) (layer F.Cu) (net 10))
 (segment (start 67.945 53.594) (end 68.794999 54.443999) (width 0.25) (layer F.Cu) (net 10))
 (segment (start 97.917 60.071) (end 99.568 58.42) (width 0.25) (layer F.Cu) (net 10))
 (segment (start 82.169 58.42) (end 83.82 60.071) (width 0.25) (layer F.Cu) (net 10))
 (segment (start 83.82 60.071) (end 97.917 60.071) (width 0.25) (layer F.Cu) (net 10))
 (segment (start 115.316 60.198) (end 117.094 58.42) (width 0.25) (layer F.Cu) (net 10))
 (segment (start 99.568 58.42) (end 101.346 60.198) (width 0.25) (layer F.Cu) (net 10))
 (segment (start 101.346 60.198) (end 115.316 60.198) (width 0.25) (layer F.Cu) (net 10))
 (segment (start 132.842 60.198) (end 134.62 58.42) (width 0.25) (layer F.Cu) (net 10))
 (segment (start 117.094 58.42) (end 118.872 60.198) (width 0.25) (layer F.Cu) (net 10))
 (segment (start 118.872 60.198) (end 132.842 60.198) (width 0.25) (layer F.Cu) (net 10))
 (segment (start 72.263 56.134) (end 74.549 58.42) (width 0.25) (layer F.Cu) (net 11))
 (segment (start 67.945 56.134) (end 72.263 56.134) (width 0.25) (layer F.Cu) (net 11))
 (segment (start 67.945 63.641002) (end 67.945 56.134) (width 0.25) (layer B.Cu) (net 11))
 (segment (start 82.709001 69.705001) (end 74.008999 69.705001) (width 0.25) (layer B.Cu) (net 11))
 (segment (start 91.948 60.466002) (end 82.709001 69.705001) (width 0.25) (layer B.Cu) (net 11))
 (segment (start 74.008999 69.705001) (end 67.945 63.641002) (width 0.25) (layer B.Cu) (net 11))
 (segment (start 91.948 58.42) (end 91.948 60.466002) (width 0.25) (layer B.Cu) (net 11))
 (segment (start 110.998 56.896) (end 109.474 58.42) (width 0.25) (layer F.Cu) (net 11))
 (segment (start 127 58.42) (end 125.476 56.896) (width 0.25) (layer F.Cu) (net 11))
 (segment (start 125.476 56.896) (end 110.998 56.896) (width 0.25) (layer F.Cu) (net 11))
 (segment (start 93.472 56.896) (end 91.948 58.42) (width 0.25) (layer F.Cu) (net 11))
 (segment (start 109.474 58.42) (end 107.95 56.896) (width 0.25) (layer F.Cu) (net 11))
 (segment (start 107.95 56.896) (end 93.472 56.896) (width 0.25) (layer F.Cu) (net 11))
 (segment (start 70.451001 83.702001) (end 95.113999 83.702001) (width 0.25) (layer B.Cu) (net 12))
 (segment (start 95.113999 83.702001) (end 96.139 82.677) (width 0.25) (layer B.Cu) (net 12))
 (segment (start 69.299 82.55) (end 70.451001 83.702001) (width 0.25) (layer B.Cu) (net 12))
 (segment (start 68.199 82.55) (end 69.299 82.55) (width 0.25) (layer B.Cu) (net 12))
 (segment (start 109.474 85.09) (end 111.887 82.677) (width 0.25) (layer B.Cu) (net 13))
 (segment (start 68.199 85.09) (end 109.474 85.09) (width 0.25) (layer B.Cu) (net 13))
 (segment (start 124.587 87.63) (end 129.667 82.55) (width 0.25) (layer B.Cu) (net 14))
 (segment (start 68.199 87.63) (end 124.587 87.63) (width 0.25) (layer B.Cu) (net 14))
 (segment (start 128.230999 89.320001) (end 135.128 82.423) (width 0.25) (layer B.Cu) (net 15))
 (segment (start 69.048999 89.320001) (end 128.230999 89.320001) (width 0.25) (layer B.Cu) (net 15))
 (segment (start 68.199 90.17) (end 69.048999 89.320001) (width 0.25) (layer B.Cu) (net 15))
 (segment (start 104.267 77.47) (end 104.267 82.677) (width 0.25) (layer F.Cu) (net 22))
 (segment (start 121.92 82.423) (end 122.047 82.55) (width 0.25) (layer F.Cu) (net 23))
 (segment (start 121.92 77.597) (end 121.92 82.423) (width 0.25) (layer F.Cu) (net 23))
 (segment (start 139.446 79.121) (end 142.748 82.423) (width 0.25) (layer F.Cu) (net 26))
 (segment (start 139.446 77.47) (end 139.446 79.121) (width 0.25) (layer F.Cu) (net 26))
 (segment (start 80 66.411) (end 82.169 68.58) (width 0.25) (layer B.Cu) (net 1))
 (segment (start 80 49.53) (end 80 66.411) (width 0.25) (layer B.Cu) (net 1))
 (segment (start 97.5 66.512) (end 99.568 68.58) (width 0.25) (layer B.Cu) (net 4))
 (segment (start 97.5 49.53) (end 97.5 66.512) (width 0.25) (layer B.Cu) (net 4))
 (segment (start 115 66.486) (end 117.094 68.58) (width 0.25) (layer B.Cu) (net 6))
 (segment (start 115 49.53) (end 115 66.486) (width 0.25) (layer B.Cu) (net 6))
 (segment (start 132.5 66.46) (end 134.62 68.58) (width 0.25) (layer B.Cu) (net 8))
 (segment (start 132.5 49.53) (end 132.5 66.46) (width 0.25) (layer B.Cu) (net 8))
 (segment (start 76.825001 48.745997) (end 76.825001 66.303999) (width 0.25) (layer B.Cu) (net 2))
 (segment (start 80 45.570998) (end 76.825001 48.745997) (width 0.25) (layer B.Cu) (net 2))
 (segment (start 76.825001 66.303999) (end 74.549 68.58) (width 0.25) (layer B.Cu) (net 2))
 (segment (start 80 43.53) (end 80 45.570998) (width 0.25) (layer B.Cu) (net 2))
 (segment (start 94.824999 65.703001) (end 91.948 68.58) (width 0.25) (layer B.Cu) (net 5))
 (segment (start 94.824999 46.205001) (end 94.824999 65.703001) (width 0.25) (layer B.Cu) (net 5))
 (segment (start 97.5 43.53) (end 94.824999 46.205001) (width 0.25) (layer B.Cu) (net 5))
 (segment (start 112.324999 65.729001) (end 109.474 68.58) (width 0.25) (layer B.Cu) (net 7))
 (segment (start 112.324999 46.205001) (end 112.324999 65.729001) (width 0.25) (layer B.Cu) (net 7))
 (segment (start 115 43.53) (end 112.324999 46.205001) (width 0.25) (layer B.Cu) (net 7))
 (segment (start 129.824999 65.755001) (end 127 68.58) (width 0.25) (layer B.Cu) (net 9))
 (segment (start 129.824999 46.205001) (end 129.824999 65.755001) (width 0.25) (layer B.Cu) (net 9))
 (segment (start 132.5 43.53) (end 129.824999 46.205001) (width 0.25) (layer B.Cu) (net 9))
 (segment (start 82.169 76.2) (end 85.725 76.2) (width 0.25) (layer B.Cu) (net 20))
 (segment (start 82.169 76.2) (end 82.169 79.756) (width 0.25) (layer F.Cu) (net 20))
 (segment (start 99.568 76.2) (end 102.997 76.2) (width 0.25) (layer B.Cu) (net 21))
 (segment (start 99.568 76.2) (end 99.568 79.629) (width 0.25) (layer F.Cu) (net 21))
 (segment (start 120.523 76.2) (end 120.65 76.327) (width 0.25) (layer B.Cu) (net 24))
 (segment (start 117.094 76.2) (end 120.523 76.2) (width 0.25) (layer B.Cu) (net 24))
 (segment (start 117.094 76.2) (end 117.094 79.629) (width 0.25) (layer F.Cu) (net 24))
 (segment (start 134.62 76.2) (end 138.176 76.2) (width 0.25) (layer B.Cu) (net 25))
 (segment (start 134.62 79.502) (end 134.366 79.756) (width 0.25) (layer F.Cu) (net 25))
 (segment (start 134.62 76.2) (end 134.62 79.502) (width 0.25) (layer F.Cu) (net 25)))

